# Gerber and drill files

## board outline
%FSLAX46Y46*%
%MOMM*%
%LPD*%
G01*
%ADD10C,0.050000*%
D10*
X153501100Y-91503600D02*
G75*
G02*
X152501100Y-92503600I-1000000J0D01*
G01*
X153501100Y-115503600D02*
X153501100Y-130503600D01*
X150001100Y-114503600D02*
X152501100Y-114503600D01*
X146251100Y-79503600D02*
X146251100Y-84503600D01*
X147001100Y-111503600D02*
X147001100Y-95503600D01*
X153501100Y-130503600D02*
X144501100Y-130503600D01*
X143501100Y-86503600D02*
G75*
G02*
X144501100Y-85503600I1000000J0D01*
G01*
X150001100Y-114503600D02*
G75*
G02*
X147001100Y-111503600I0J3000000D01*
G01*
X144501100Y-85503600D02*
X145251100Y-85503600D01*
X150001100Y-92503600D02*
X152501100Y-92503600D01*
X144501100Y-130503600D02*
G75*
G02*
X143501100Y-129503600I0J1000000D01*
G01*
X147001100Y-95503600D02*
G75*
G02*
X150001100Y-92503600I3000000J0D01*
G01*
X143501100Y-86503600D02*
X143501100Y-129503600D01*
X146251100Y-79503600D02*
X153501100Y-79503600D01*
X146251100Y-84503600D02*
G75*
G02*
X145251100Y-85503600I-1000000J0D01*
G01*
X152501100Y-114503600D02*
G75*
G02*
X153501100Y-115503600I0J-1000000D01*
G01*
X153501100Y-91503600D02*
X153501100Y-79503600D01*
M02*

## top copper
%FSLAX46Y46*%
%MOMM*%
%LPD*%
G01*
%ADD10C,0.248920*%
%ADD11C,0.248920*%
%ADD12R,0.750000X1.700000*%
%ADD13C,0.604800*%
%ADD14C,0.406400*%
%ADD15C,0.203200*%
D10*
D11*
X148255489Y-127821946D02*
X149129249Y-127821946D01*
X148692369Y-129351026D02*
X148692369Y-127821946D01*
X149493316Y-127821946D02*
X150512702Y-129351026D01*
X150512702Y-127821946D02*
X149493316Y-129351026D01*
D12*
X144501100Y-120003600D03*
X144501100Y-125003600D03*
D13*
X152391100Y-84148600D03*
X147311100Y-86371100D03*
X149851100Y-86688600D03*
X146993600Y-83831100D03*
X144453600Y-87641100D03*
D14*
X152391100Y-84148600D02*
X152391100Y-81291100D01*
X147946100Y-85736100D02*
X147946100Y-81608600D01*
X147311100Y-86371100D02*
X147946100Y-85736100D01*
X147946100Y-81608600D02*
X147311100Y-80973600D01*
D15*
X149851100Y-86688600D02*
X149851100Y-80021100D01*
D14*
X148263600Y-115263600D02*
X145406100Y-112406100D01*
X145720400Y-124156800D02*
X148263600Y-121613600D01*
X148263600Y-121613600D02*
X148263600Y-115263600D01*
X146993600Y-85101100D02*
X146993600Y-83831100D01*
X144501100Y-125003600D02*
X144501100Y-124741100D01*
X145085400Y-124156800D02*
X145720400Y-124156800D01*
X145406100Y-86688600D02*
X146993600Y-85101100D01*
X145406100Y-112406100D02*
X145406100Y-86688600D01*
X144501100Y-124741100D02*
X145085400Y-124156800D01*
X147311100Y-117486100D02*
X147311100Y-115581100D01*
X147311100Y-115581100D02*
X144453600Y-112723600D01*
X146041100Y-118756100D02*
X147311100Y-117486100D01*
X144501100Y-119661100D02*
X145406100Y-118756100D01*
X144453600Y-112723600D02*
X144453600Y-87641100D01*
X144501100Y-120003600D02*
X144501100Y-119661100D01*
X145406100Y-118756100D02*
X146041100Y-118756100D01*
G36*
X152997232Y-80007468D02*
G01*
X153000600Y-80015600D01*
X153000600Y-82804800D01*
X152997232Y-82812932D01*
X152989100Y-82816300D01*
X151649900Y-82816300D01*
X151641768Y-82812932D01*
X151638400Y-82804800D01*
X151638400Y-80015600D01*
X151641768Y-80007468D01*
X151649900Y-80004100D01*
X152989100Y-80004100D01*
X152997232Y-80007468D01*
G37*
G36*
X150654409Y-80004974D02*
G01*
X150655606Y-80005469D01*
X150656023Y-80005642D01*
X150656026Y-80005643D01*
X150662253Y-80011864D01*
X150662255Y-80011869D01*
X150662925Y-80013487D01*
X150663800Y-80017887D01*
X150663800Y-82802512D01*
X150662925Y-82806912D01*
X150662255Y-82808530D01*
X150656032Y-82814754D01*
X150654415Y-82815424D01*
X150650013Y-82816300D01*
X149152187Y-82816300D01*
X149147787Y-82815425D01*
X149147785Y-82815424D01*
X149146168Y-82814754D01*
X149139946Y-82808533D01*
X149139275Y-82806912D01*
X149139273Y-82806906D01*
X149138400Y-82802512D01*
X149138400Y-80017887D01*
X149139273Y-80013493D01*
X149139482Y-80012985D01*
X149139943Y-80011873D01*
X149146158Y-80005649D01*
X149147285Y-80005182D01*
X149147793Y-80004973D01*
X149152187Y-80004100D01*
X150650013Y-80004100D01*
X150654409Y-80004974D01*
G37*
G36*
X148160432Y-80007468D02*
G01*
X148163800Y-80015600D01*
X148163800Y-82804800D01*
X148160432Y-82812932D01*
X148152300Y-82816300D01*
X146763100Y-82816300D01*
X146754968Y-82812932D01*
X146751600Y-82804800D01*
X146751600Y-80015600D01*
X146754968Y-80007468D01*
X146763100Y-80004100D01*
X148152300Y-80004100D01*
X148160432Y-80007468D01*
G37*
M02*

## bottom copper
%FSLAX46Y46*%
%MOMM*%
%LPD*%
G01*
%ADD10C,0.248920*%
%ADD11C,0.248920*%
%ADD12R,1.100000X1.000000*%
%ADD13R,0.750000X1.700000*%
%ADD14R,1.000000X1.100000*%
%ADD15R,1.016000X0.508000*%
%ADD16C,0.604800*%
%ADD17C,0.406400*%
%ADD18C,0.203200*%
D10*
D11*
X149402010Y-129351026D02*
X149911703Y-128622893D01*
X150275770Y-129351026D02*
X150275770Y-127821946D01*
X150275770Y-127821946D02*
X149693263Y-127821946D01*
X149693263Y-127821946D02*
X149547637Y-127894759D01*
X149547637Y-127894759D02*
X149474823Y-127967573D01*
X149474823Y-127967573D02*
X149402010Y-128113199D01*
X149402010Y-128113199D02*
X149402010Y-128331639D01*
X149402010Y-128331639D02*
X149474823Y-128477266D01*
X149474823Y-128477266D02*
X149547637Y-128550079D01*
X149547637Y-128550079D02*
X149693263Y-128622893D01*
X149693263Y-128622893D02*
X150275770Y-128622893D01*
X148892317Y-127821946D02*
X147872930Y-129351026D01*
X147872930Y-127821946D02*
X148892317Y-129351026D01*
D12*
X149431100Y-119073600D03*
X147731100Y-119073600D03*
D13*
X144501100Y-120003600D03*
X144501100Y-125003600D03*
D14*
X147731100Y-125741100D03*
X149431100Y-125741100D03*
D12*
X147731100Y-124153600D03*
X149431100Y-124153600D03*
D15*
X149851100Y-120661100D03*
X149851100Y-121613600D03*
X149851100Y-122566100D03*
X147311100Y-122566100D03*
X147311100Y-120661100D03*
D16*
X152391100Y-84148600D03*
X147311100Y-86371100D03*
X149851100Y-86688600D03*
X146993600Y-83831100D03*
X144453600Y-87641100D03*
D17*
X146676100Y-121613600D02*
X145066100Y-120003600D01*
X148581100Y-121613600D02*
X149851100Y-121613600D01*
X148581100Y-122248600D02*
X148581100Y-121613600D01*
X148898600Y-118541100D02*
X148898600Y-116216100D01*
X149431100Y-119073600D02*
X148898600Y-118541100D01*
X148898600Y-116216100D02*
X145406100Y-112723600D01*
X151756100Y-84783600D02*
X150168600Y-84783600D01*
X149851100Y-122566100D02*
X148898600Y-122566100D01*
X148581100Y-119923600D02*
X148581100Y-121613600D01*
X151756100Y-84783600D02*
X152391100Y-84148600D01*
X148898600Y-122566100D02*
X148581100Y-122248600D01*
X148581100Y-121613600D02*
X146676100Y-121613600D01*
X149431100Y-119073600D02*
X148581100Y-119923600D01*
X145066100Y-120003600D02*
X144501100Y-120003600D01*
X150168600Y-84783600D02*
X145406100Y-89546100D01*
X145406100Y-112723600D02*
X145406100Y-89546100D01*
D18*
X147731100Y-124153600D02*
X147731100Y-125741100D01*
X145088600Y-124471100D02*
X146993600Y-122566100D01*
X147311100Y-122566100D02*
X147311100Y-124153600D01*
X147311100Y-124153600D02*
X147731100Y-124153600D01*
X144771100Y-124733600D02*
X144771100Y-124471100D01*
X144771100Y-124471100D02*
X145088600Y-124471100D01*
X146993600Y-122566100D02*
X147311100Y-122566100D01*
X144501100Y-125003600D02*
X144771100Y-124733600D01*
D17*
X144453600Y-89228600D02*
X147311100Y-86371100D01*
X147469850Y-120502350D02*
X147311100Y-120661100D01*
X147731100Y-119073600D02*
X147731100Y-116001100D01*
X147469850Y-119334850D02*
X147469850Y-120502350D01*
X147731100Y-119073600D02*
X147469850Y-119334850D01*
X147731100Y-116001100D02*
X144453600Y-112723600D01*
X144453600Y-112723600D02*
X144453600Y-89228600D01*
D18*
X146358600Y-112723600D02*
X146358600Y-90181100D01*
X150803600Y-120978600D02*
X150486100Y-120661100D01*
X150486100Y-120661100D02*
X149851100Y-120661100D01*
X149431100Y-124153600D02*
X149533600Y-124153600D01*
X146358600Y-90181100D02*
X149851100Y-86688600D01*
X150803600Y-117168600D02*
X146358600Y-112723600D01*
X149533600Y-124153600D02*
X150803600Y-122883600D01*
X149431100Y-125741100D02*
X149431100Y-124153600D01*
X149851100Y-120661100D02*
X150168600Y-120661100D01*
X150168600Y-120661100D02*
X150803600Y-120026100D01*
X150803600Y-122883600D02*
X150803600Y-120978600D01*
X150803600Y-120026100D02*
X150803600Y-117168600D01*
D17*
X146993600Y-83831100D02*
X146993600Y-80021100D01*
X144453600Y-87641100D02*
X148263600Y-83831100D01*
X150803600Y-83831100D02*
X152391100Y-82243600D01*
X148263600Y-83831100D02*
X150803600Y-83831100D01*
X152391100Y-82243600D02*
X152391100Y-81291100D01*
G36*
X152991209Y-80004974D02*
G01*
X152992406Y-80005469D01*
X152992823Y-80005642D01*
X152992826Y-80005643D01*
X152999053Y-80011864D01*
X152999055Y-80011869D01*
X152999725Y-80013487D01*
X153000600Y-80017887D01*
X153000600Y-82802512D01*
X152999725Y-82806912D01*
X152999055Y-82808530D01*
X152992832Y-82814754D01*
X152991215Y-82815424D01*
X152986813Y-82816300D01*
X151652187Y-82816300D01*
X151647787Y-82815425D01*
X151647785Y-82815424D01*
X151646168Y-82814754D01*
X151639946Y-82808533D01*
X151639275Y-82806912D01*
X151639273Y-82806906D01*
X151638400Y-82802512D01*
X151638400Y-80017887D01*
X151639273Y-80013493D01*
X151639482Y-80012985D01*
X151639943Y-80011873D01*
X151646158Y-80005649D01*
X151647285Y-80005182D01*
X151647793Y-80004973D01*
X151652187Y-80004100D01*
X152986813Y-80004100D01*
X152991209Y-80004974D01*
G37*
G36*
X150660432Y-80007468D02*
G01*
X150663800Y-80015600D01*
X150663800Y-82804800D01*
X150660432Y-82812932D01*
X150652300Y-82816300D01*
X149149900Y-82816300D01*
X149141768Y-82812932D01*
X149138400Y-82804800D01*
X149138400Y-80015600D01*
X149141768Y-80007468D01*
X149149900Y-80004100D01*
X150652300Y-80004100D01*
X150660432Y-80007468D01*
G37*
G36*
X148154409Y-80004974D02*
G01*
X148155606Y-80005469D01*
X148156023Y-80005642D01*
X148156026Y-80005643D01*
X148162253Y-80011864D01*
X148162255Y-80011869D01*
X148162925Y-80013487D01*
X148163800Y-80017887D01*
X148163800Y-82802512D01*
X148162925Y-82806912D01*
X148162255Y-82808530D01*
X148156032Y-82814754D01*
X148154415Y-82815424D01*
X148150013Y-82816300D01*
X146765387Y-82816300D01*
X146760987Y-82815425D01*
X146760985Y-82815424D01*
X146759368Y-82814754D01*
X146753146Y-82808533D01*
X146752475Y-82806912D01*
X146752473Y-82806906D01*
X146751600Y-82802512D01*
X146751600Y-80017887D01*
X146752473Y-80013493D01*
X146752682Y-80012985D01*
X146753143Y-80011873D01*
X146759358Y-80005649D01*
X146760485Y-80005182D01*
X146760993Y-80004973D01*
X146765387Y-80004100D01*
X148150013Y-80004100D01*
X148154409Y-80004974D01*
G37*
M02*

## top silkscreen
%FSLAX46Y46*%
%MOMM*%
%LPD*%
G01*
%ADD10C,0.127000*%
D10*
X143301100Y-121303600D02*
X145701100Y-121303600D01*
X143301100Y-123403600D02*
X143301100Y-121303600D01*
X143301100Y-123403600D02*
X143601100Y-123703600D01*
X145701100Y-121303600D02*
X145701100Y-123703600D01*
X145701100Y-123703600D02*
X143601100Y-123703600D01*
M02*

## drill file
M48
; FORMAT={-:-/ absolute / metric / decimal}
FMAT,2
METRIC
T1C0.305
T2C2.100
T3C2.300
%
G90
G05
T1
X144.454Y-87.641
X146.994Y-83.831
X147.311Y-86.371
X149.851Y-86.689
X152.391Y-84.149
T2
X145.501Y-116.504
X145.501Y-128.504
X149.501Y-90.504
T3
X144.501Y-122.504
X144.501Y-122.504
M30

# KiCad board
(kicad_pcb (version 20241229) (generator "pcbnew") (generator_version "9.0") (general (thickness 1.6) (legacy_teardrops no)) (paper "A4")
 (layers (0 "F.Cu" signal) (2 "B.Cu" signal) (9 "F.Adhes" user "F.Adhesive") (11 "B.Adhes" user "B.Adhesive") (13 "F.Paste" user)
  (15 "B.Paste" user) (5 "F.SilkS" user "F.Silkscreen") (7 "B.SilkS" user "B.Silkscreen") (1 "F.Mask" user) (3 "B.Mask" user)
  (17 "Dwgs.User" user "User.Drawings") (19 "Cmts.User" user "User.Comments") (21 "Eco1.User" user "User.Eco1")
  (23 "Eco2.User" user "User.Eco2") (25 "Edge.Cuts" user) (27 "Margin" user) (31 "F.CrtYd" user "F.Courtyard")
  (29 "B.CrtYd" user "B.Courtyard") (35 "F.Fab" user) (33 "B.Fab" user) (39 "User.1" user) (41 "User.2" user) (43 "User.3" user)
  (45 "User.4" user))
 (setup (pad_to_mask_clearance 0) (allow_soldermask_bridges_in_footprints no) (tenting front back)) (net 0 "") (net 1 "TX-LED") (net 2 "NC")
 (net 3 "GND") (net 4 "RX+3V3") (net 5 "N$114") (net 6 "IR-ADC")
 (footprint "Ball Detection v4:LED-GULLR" (layer "F.Cu") (at 144.5011 122.5036 90)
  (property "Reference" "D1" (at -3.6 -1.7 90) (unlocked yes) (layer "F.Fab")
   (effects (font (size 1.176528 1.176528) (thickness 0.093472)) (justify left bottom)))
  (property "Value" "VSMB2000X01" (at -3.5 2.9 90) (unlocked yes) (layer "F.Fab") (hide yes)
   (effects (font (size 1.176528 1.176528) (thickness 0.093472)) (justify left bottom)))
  (fp_line (start 1.2 -1.2) (end 1.2 1.2) (stroke (width 0.127) (type solid)) (layer "F.SilkS"))
  (fp_line (start -0.9 -1.2) (end 1.2 -1.2) (stroke (width 0.127) (type solid)) (layer "F.SilkS"))
  (fp_line (start -0.9 -1.2) (end -1.2 -0.9) (stroke (width 0.127) (type solid)) (layer "F.SilkS"))
  (fp_line (start 1.2 1.2) (end -1.2 1.2) (stroke (width 0.127) (type solid)) (layer "F.SilkS"))
  (fp_line (start -1.2 1.2) (end -1.2 -0.9) (stroke (width 0.127) (type solid)) (layer "F.SilkS"))
  (pad "" np_thru_hole circle (at 0 0 90) (size 2.3 2.3) (drill 2.3) (layers "*.Cu" "*.Mask"))
  (pad "A" smd rect (at 2.5 0 90) (size 1.7 0.75) (layers "F.Cu" "F.Mask" "F.Paste") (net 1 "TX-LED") (solder_mask_margin 0.075)
   (solder_paste_margin 0) (thermal_bridge_angle 0))
  (pad "C" smd rect (at -2.5 0 90) (size 1.7 0.75) (layers "F.Cu" "F.Mask" "F.Paste") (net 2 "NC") (solder_mask_margin 0.075)
   (solder_paste_margin 0) (thermal_bridge_angle 0)))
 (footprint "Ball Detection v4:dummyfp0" (layer "F.Cu") (at 145.5011 128.5036)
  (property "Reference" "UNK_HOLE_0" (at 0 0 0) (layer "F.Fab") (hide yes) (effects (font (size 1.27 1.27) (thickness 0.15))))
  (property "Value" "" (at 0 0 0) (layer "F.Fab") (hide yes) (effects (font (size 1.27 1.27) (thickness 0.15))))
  (pad "" np_thru_hole circle (at 0 0) (size 2.1 2.1) (drill 2.1) (layers "*.Cu" "*.Mask")))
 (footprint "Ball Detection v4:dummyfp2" (layer "F.Cu") (at 149.5011 90.5036)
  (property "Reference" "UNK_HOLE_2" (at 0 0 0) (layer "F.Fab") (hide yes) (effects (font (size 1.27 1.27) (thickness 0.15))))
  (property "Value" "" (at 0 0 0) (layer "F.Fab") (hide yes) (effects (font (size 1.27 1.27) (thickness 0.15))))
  (pad "" np_thru_hole circle (at 0 0) (size 2.1 2.1) (drill 2.1) (layers "*.Cu" "*.Mask")))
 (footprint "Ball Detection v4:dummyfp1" (layer "F.Cu") (at 145.5011 116.5036)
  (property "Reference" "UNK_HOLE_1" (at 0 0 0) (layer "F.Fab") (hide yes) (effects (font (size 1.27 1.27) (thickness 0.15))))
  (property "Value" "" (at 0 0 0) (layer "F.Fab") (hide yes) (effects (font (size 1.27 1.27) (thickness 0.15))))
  (pad "" np_thru_hole circle (at 0 0) (size 2.1 2.1) (drill 2.1) (layers "*.Cu" "*.Mask")))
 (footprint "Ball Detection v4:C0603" (layer "B.Cu") (at 148.5811 119.0736 180)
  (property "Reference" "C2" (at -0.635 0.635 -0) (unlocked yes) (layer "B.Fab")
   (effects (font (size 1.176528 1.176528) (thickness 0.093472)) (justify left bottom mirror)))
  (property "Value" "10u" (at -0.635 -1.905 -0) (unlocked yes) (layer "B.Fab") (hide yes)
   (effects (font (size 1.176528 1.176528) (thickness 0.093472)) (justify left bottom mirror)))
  (pad "1" smd rect (at -0.85 0 180) (size 1.1 1) (layers "B.Cu" "B.Mask" "B.Paste") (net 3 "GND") (solder_mask_margin 0.075)
   (solder_paste_margin 0) (thermal_bridge_angle 0))
  (pad "2" smd rect (at 0.85 0 180) (size 1.1 1) (layers "B.Cu" "B.Mask" "B.Paste") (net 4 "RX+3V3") (solder_mask_margin 0.075)
   (solder_paste_margin 0) (thermal_bridge_angle 0)))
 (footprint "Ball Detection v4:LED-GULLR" (layer "B.Cu") (at 144.5011 122.5036 90)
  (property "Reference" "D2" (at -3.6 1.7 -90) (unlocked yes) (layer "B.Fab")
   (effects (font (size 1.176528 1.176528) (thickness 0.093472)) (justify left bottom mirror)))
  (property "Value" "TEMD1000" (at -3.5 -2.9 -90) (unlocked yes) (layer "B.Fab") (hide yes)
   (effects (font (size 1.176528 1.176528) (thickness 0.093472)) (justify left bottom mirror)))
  (pad "" np_thru_hole circle (at 0 0 90) (size 2.3 2.3) (drill 2.3) (layers "*.Cu" "*.Mask"))
  (pad "A" smd rect (at 2.5 0 90) (size 1.7 0.75) (layers "B.Cu" "B.Mask" "B.Paste") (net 3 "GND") (solder_mask_margin 0.075)
   (solder_paste_margin 0) (thermal_bridge_angle 0))
  (pad "C" smd rect (at -2.5 0 90) (size 1.7 0.75) (layers "B.Cu" "B.Mask" "B.Paste") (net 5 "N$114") (solder_mask_margin 0.075)
   (solder_paste_margin 0) (thermal_bridge_angle 0)))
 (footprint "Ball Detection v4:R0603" (layer "B.Cu") (at 148.5811 125.7411)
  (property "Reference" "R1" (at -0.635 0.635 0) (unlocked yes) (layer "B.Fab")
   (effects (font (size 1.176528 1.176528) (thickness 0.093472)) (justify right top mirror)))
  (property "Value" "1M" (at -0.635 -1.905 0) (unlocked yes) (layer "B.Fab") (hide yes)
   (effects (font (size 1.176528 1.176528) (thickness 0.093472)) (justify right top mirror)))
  (pad "1" smd rect (at -0.85 0) (size 1 1.1) (layers "B.Cu" "B.Mask" "B.Paste") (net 5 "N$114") (solder_mask_margin 0.075)
   (solder_paste_margin 0) (thermal_bridge_angle 0))
  (pad "2" smd rect (at 0.85 0) (size 1 1.1) (layers "B.Cu" "B.Mask" "B.Paste") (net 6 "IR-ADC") (solder_mask_margin 0.075)
   (solder_paste_margin 0) (thermal_bridge_angle 0)))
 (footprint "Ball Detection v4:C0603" (layer "B.Cu") (at 148.5811 124.1536)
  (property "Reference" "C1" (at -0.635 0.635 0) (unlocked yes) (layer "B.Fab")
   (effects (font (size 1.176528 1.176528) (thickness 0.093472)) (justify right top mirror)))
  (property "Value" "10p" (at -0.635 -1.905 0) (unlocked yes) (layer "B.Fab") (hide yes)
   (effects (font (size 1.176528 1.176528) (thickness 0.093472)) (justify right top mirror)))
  (pad "1" smd rect (at -0.85 0) (size 1.1 1) (layers "B.Cu" "B.Mask" "B.Paste") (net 5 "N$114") (solder_mask_margin 0.075)
   (solder_paste_margin 0) (thermal_bridge_angle 0))
  (pad "2" smd rect (at 0.85 0) (size 1.1 1) (layers "B.Cu" "B.Mask" "B.Paste") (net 6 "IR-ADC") (solder_mask_margin 0.075)
   (solder_paste_margin 0) (thermal_bridge_angle 0)))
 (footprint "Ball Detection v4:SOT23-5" (layer "B.Cu") (at 148.5811 121.6136 180)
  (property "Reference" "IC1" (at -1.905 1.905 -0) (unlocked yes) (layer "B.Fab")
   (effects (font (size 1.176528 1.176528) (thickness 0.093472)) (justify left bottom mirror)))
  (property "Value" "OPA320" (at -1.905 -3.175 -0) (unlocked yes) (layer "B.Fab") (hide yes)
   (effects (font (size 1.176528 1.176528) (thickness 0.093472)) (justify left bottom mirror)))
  (pad "1" smd rect (at -1.27 0.9525 180) (size 1.016 0.508) (layers "B.Cu" "B.Mask" "B.Paste") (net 6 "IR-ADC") (solder_mask_margin 0.075)
   (solder_paste_margin 0) (thermal_bridge_angle 0))
  (pad "2" smd rect (at -1.27 0 180) (size 1.016 0.508) (layers "B.Cu" "B.Mask" "B.Paste") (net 3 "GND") (solder_mask_margin 0.075)
   (solder_paste_margin 0) (thermal_bridge_angle 0))
  (pad "3" smd rect (at -1.27 -0.9525 180) (size 1.016 0.508) (layers "B.Cu" "B.Mask" "B.Paste") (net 3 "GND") (solder_mask_margin 0.075)
   (solder_paste_margin 0) (thermal_bridge_angle 0))
  (pad "4" smd rect (at 1.27 -0.9525 180) (size 1.016 0.508) (layers "B.Cu" "B.Mask" "B.Paste") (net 5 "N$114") (solder_mask_margin 0.075)
   (solder_paste_margin 0) (thermal_bridge_angle 0))
  (pad "5" smd rect (at 1.27 0.9525 180) (size 1.016 0.508) (layers "B.Cu" "B.Mask" "B.Paste") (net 4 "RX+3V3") (solder_mask_margin 0.075)
   (solder_paste_margin 0) (thermal_bridge_angle 0)))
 (gr_arc (start 153.5011 91.5036) (mid 153.208207 92.210707) (end 152.5011 92.5036) (stroke (width 0.05) (type solid)) (layer "Edge.Cuts"))
 (gr_line (start 153.5011 115.5036) (end 153.5011 130.5036) (stroke (width 0.05) (type solid)) (layer "Edge.Cuts"))
 (gr_line (start 150.0011 114.5036) (end 152.5011 114.5036) (stroke (width 0.05) (type solid)) (layer "Edge.Cuts"))
 (gr_line (start 146.2511 79.5036) (end 146.2511 84.5036) (stroke (width 0.05) (type solid)) (layer "Edge.Cuts"))
 (gr_line (start 147.0011 111.5036) (end 147.0011 95.5036) (stroke (width 0.05) (type solid)) (layer "Edge.Cuts"))
 (gr_line (start 153.5011 130.5036) (end 144.5011 130.5036) (stroke (width 0.05) (type solid)) (layer "Edge.Cuts"))
 (gr_arc (start 143.5011 86.5036) (mid 143.793993 85.796493) (end 144.5011 85.5036) (stroke (width 0.05) (type solid)) (layer "Edge.Cuts"))
 (gr_arc (start 150.0011 114.5036) (mid 147.87978 113.62492) (end 147.0011 111.5036) (stroke (width 0.05) (type solid)) (layer "Edge.Cuts"))
 (gr_line (start 144.5011 85.5036) (end 145.2511 85.5036) (stroke (width 0.05) (type solid)) (layer "Edge.Cuts"))
 (gr_line (start 150.0011 92.5036) (end 152.5011 92.5036) (stroke (width 0.05) (type solid)) (layer "Edge.Cuts"))
 (gr_arc (start 144.5011 130.5036) (mid 143.793993 130.210707) (end 143.5011 129.5036) (stroke (width 0.05) (type solid))
  (layer "Edge.Cuts"))
 (gr_arc (start 147.0011 95.5036) (mid 147.87978 93.38228) (end 150.0011 92.5036) (stroke (width 0.05) (type solid)) (layer "Edge.Cuts"))
 (gr_line (start 143.5011 86.5036) (end 143.5011 129.5036) (stroke (width 0.05) (type solid)) (layer "Edge.Cuts"))
 (gr_line (start 146.2511 79.5036) (end 153.5011 79.5036) (stroke (width 0.05) (type solid)) (layer "Edge.Cuts"))
 (gr_arc (start 146.2511 84.5036) (mid 145.958207 85.210707) (end 145.2511 85.5036) (stroke (width 0.05) (type solid)) (layer "Edge.Cuts"))
 (gr_arc (start 152.5011 114.5036) (mid 153.208207 114.796493) (end 153.5011 115.5036) (stroke (width 0.05) (type solid))
  (layer "Edge.Cuts"))
 (gr_line (start 153.5011 91.5036) (end 153.5011 79.5036) (stroke (width 0.05) (type solid)) (layer "Edge.Cuts"))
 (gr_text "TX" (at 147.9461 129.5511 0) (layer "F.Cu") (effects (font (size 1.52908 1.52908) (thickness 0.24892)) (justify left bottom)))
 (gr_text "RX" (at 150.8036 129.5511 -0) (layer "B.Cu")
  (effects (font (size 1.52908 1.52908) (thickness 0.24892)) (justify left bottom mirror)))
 (segment (start 152.3911 84.1486) (end 152.3911 81.2911) (width 0.4064) (layer "F.Cu") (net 3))
 (via (at 152.3911 84.1486) (size 0.6048) (drill 0.3048) (layers "F.Cu" "B.Cu") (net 3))
 (segment (start 146.6761 121.6136) (end 145.0661 120.0036) (width 0.4064) (layer "B.Cu") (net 3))
 (segment (start 148.5811 121.6136) (end 149.8511 121.6136) (width 0.4064) (layer "B.Cu") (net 3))
 (segment (start 148.5811 122.2486) (end 148.5811 121.6136) (width 0.4064) (layer "B.Cu") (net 3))
 (segment (start 148.8986 118.5411) (end 148.8986 116.2161) (width 0.4064) (layer "B.Cu") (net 3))
 (segment (start 149.4311 119.0736) (end 148.8986 118.5411) (width 0.4064) (layer "B.Cu") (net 3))
 (segment (start 148.8986 116.2161) (end 145.4061 112.7236) (width 0.4064) (layer "B.Cu") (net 3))
 (segment (start 151.7561 84.7836) (end 150.1686 84.7836) (width 0.4064) (layer "B.Cu") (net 3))
 (segment (start 149.8511 122.5661) (end 148.8986 122.5661) (width 0.4064) (layer "B.Cu") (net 3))
 (segment (start 148.5811 119.9236) (end 148.5811 121.6136) (width 0.4064) (layer "B.Cu") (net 3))
 (segment (start 151.7561 84.7836) (end 152.3911 84.1486) (width 0.4064) (layer "B.Cu") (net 3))
 (segment (start 148.8986 122.5661) (end 148.5811 122.2486) (width 0.4064) (layer "B.Cu") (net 3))
 (segment (start 148.5811 121.6136) (end 146.6761 121.6136) (width 0.4064) (layer "B.Cu") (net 3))
 (segment (start 149.4311 119.0736) (end 148.5811 119.9236) (width 0.4064) (layer "B.Cu") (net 3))
 (segment (start 145.0661 120.0036) (end 144.5011 120.0036) (width 0.4064) (layer "B.Cu") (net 3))
 (segment (start 150.1686 84.7836) (end 145.4061 89.5461) (width 0.4064) (layer "B.Cu") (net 3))
 (segment (start 145.4061 112.7236) (end 145.4061 89.5461) (width 0.4064) (layer "B.Cu") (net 3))
 (segment (start 147.7311 124.1536) (end 147.7311 125.7411) (width 0.2032) (layer "B.Cu") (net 5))
 (segment (start 145.0886 124.4711) (end 146.9936 122.5661) (width 0.2032) (layer "B.Cu") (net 5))
 (segment (start 147.3111 122.5661) (end 147.3111 124.1536) (width 0.2032) (layer "B.Cu") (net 5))
 (segment (start 147.3111 124.1536) (end 147.7311 124.1536) (width 0.2032) (layer "B.Cu") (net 5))
 (segment (start 144.7711 124.7336) (end 144.7711 124.4711) (width 0.2032) (layer "B.Cu") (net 5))
 (segment (start 144.7711 124.4711) (end 145.0886 124.4711) (width 0.2032) (layer "B.Cu") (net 5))
 (segment (start 146.9936 122.5661) (end 147.3111 122.5661) (width 0.2032) (layer "B.Cu") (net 5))
 (segment (start 144.5011 125.0036) (end 144.7711 124.7336) (width 0.2032) (layer "B.Cu") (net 5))
 (segment (start 147.9461 85.7361) (end 147.9461 81.6086) (width 0.4064) (layer "F.Cu") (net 4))
 (segment (start 147.3111 86.3711) (end 147.9461 85.7361) (width 0.4064) (layer "F.Cu") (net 4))
 (segment (start 147.9461 81.6086) (end 147.3111 80.9736) (width 0.4064) (layer "F.Cu") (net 4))
 (via (at 147.3111 86.3711) (size 0.6048) (drill 0.3048) (layers "F.Cu" "B.Cu") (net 4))
 (segment (start 144.4536 89.2286) (end 147.3111 86.3711) (width 0.4064) (layer "B.Cu") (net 4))
 (segment (start 147.46985 120.50235) (end 147.3111 120.6611) (width 0.4064) (layer "B.Cu") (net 4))
 (segment (start 147.7311 119.0736) (end 147.7311 116.0011) (width 0.4064) (layer "B.Cu") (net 4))
 (segment (start 147.46985 119.33485) (end 147.46985 120.50235) (width 0.4064) (layer "B.Cu") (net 4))
 (segment (start 147.7311 119.0736) (end 147.46985 119.33485) (width 0.4064) (layer "B.Cu") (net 4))
 (segment (start 147.7311 116.0011) (end 144.4536 112.7236) (width 0.4064) (layer "B.Cu") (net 4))
 (segment (start 144.4536 112.7236) (end 144.4536 89.2286) (width 0.4064) (layer "B.Cu") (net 4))
 (segment (start 149.8511 86.6886) (end 149.8511 80.0211) (width 0.2032) (layer "F.Cu") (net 6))
 (via (at 149.8511 86.6886) (size 0.6048) (drill 0.3048) (layers "F.Cu" "B.Cu") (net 6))
 (segment (start 146.3586 112.7236) (end 146.3586 90.1811) (width 0.2032) (layer "B.Cu") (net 6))
 (segment (start 150.8036 120.9786) (end 150.4861 120.6611) (width 0.2032) (layer "B.Cu") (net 6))
 (segment (start 150.4861 120.6611) (end 149.8511 120.6611) (width 0.2032) (layer "B.Cu") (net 6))
 (segment (start 149.4311 124.1536) (end 149.5336 124.1536) (width 0.2032) (layer "B.Cu") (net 6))
 (segment (start 146.3586 90.1811) (end 149.8511 86.6886) (width 0.2032) (layer "B.Cu") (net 6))
 (segment (start 150.8036 117.1686) (end 146.3586 112.7236) (width 0.2032) (layer "B.Cu") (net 6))
 (segment (start 149.5336 124.1536) (end 150.8036 122.8836) (width 0.2032) (layer "B.Cu") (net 6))
 (segment (start 149.4311 125.7411) (end 149.4311 124.1536) (width 0.2032) (layer "B.Cu") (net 6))
 (segment (start 149.8511 120.6611) (end 150.1686 120.6611) (width 0.2032) (layer "B.Cu") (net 6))
 (segment (start 150.1686 120.6611) (end 150.8036 120.0261) (width 0.2032) (layer "B.Cu") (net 6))
 (segment (start 150.8036 122.8836) (end 150.8036 120.9786) (width 0.2032) (layer "B.Cu") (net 6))
 (segment (start 150.8036 120.0261) (end 150.8036 117.1686) (width 0.2032) (layer "B.Cu") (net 6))
 (segment (start 148.2636 115.2636) (end 145.4061 112.4061) (width 0.4064) (layer "F.Cu") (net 2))
 (segment (start 145.7204 124.1568) (end 148.2636 121.6136) (width 0.4064) (layer "F.Cu") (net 2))
 (segment (start 148.2636 121.6136) (end 148.2636 115.2636) (width 0.4064) (layer "F.Cu") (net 2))
 (segment (start 146.9936 85.1011) (end 146.9936 83.8311) (width 0.4064) (layer "F.Cu") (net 2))
 (segment (start 144.5011 125.0036) (end 144.5011 124.7411) (width 0.4064) (layer "F.Cu") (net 2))
 (segment (start 145.0854 124.1568) (end 145.7204 124.1568) (width 0.4064) (layer "F.Cu") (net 2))
 (segment (start 145.4061 86.6886) (end 146.9936 85.1011) (width 0.4064) (layer "F.Cu") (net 2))
 (segment (start 145.4061 112.4061) (end 145.4061 86.6886) (width 0.4064) (layer "F.Cu") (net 2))
 (segment (start 144.5011 124.7411) (end 145.0854 124.1568) (width 0.4064) (layer "F.Cu") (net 2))
 (via (at 146.9936 83.8311) (size 0.6048) (drill 0.3048) (layers "F.Cu" "B.Cu") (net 2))
 (segment (start 146.9936 83.8311) (end 146.9936 80.0211) (width 0.4064) (layer "B.Cu") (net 2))
 (segment (start 147.3111 117.4861) (end 147.3111 115.5811) (width 0.4064) (layer "F.Cu") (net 1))
 (segment (start 147.3111 115.5811) (end 144.4536 112.7236) (width 0.4064) (layer "F.Cu") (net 1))
 (segment (start 146.0411 118.7561) (end 147.3111 117.4861) (width 0.4064) (layer "F.Cu") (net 1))
 (segment (start 144.5011 119.6611) (end 145.4061 118.7561) (width 0.4064) (layer "F.Cu") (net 1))
 (segment (start 144.4536 112.7236) (end 144.4536 87.6411) (width 0.4064) (layer "F.Cu") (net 1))
 (segment (start 144.5011 120.0036) (end 144.5011 119.6611) (width 0.4064) (layer "F.Cu") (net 1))
 (segment (start 145.4061 118.7561) (end 146.0411 118.7561) (width 0.4064) (layer "F.Cu") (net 1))
 (via (at 144.4536 87.6411) (size 0.6048) (drill 0.3048) (layers "F.Cu" "B.Cu") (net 1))
 (segment (start 144.4536 87.6411) (end 148.2636 83.8311) (width 0.4064) (layer "B.Cu") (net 1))
 (segment (start 150.8036 83.8311) (end 152.3911 82.2436) (width 0.4064) (layer "B.Cu") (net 1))
 (segment (start 148.2636 83.8311) (end 150.8036 83.8311) (width 0.4064) (layer "B.Cu") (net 1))
 (segment (start 152.3911 82.2436) (end 152.3911 81.2911) (width 0.4064) (layer "B.Cu") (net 1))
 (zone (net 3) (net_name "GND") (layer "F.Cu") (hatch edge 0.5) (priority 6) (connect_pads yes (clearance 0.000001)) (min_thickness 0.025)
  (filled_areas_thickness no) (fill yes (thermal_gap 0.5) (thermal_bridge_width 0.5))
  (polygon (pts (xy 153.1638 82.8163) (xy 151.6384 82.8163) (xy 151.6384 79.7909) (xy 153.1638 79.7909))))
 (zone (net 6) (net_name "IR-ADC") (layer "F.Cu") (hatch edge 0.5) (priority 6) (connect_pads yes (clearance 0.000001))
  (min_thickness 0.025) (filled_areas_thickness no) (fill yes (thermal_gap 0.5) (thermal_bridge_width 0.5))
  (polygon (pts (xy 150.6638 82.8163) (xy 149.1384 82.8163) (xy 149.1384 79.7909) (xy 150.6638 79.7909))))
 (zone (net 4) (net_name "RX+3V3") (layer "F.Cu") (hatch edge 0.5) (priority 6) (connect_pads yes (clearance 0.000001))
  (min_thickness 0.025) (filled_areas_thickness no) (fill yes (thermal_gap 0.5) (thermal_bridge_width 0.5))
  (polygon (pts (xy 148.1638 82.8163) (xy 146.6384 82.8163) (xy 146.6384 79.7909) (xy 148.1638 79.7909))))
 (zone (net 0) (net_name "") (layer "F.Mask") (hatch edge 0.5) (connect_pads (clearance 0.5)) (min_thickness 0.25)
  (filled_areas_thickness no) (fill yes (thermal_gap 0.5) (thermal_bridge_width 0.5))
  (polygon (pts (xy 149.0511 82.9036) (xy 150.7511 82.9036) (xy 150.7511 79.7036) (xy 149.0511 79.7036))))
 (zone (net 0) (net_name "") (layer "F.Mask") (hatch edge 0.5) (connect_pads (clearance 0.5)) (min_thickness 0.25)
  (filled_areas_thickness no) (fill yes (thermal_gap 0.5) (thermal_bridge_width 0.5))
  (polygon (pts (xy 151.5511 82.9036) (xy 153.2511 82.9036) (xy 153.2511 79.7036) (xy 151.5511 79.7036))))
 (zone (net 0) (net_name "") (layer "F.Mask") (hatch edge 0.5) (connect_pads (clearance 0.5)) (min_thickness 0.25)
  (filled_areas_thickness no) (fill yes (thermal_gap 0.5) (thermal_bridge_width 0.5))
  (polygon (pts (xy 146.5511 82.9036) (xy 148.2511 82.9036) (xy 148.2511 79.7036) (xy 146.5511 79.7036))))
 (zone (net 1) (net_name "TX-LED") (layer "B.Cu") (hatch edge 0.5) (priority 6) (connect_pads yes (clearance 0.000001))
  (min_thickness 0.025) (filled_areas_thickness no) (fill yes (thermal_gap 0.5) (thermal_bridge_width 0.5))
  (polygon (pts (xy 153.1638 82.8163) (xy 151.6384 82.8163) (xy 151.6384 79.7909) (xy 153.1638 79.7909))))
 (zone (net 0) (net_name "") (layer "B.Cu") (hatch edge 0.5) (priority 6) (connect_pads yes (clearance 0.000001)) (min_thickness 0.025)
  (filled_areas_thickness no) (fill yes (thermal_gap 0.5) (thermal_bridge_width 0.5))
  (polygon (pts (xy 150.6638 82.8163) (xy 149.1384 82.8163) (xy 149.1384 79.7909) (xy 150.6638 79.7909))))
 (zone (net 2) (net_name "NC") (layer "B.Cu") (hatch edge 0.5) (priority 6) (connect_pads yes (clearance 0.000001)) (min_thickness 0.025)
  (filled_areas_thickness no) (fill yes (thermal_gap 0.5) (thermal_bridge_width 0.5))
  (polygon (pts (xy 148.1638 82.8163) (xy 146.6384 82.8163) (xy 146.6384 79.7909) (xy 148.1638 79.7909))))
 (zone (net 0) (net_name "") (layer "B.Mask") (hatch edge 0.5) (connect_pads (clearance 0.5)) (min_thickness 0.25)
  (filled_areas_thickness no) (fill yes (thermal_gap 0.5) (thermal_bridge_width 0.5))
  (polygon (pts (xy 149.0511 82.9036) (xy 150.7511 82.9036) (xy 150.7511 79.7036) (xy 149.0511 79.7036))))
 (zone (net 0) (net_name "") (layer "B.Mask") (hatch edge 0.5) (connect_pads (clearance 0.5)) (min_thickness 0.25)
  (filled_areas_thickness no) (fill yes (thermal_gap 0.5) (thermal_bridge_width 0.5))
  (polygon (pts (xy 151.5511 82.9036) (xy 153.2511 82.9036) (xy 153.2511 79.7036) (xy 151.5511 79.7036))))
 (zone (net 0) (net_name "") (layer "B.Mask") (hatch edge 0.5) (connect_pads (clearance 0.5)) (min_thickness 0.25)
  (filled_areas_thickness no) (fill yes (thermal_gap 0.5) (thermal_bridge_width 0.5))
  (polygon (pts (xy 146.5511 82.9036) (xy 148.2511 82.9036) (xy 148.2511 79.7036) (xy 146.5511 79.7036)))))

